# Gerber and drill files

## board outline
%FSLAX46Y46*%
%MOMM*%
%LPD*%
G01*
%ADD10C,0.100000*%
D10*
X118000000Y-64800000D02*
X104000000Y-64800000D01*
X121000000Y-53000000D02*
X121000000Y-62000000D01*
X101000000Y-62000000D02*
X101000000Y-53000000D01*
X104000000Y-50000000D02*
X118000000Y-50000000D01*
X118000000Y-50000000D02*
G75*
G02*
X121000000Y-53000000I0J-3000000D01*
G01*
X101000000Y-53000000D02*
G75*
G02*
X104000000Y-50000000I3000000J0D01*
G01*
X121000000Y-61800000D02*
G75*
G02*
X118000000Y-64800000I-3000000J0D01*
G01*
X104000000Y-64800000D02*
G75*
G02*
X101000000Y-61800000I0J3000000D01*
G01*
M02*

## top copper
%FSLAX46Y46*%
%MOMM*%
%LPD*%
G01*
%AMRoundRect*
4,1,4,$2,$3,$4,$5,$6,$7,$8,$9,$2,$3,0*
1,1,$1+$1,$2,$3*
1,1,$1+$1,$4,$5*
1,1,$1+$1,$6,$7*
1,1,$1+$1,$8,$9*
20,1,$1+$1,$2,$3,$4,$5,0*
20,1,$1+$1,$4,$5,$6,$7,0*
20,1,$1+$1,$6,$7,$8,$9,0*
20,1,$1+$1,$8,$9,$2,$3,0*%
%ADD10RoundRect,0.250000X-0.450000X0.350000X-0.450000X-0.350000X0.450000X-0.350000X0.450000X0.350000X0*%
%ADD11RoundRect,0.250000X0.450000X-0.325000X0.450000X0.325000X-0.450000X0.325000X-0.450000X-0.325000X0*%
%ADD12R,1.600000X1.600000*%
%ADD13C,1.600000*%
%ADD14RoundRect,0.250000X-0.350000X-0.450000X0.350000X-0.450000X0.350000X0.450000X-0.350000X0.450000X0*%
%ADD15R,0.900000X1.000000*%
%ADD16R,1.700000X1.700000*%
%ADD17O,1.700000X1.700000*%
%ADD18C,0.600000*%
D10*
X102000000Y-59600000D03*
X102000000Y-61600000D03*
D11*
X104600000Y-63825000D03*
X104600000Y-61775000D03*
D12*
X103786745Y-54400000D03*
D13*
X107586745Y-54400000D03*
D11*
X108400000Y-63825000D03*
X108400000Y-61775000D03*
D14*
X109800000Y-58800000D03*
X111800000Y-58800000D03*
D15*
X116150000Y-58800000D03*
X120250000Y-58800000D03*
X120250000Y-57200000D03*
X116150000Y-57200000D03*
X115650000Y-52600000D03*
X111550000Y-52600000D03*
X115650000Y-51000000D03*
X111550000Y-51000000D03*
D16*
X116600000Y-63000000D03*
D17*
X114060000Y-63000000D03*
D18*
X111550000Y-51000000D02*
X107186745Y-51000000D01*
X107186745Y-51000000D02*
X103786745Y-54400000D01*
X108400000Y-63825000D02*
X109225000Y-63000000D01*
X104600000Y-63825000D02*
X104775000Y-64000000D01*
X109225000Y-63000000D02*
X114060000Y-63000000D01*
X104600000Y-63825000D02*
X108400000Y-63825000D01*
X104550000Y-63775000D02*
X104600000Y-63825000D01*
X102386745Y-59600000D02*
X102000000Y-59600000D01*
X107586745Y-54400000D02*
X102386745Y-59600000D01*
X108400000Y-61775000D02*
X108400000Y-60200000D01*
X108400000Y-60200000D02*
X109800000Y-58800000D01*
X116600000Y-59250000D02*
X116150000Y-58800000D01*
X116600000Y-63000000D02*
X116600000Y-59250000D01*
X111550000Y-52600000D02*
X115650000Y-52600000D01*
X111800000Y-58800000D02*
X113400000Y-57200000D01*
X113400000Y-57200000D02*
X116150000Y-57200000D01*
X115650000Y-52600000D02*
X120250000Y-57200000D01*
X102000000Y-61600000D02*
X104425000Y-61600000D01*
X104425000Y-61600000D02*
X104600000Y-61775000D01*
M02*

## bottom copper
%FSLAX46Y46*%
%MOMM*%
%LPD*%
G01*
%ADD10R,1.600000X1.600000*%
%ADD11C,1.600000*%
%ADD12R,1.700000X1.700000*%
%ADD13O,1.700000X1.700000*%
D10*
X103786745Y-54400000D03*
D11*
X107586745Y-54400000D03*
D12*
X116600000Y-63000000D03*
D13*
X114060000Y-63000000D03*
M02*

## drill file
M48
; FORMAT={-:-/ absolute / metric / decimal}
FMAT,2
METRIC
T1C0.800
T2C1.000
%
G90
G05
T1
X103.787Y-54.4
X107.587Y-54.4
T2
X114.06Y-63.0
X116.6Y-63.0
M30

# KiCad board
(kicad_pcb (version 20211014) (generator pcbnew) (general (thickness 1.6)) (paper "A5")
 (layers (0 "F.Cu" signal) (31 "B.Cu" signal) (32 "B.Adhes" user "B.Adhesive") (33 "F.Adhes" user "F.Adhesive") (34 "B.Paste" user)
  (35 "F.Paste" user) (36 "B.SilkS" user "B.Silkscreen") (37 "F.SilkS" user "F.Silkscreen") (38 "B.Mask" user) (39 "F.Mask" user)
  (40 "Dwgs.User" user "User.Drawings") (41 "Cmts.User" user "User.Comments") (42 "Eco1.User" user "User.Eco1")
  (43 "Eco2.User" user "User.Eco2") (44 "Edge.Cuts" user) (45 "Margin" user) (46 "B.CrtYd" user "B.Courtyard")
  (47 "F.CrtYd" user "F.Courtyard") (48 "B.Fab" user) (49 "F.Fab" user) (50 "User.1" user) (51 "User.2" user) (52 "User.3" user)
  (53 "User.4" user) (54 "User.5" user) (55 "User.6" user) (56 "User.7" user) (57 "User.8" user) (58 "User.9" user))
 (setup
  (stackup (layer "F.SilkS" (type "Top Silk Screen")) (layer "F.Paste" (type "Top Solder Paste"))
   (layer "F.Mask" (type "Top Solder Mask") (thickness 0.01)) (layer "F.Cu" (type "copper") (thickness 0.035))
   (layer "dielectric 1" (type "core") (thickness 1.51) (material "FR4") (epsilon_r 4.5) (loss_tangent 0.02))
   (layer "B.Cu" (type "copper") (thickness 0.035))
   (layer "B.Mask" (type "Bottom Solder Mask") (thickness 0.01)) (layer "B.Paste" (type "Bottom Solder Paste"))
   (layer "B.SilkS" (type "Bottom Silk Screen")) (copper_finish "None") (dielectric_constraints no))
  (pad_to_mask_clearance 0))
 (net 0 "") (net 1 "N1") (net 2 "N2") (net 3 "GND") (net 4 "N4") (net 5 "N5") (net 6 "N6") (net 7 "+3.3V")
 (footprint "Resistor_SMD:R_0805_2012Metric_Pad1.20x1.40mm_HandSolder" (layer "F.Cu") (at 102 60.6 -90)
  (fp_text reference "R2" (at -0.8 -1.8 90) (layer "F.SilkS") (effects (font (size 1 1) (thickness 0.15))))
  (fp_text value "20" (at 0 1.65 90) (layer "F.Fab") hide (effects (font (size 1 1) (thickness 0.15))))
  (pad "1" smd roundrect (at -1 0 270) (size 1.2 1.4) (layers "F.Cu" "F.Paste" "F.Mask") (roundrect_rratio 0.208333) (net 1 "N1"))
  (pad "2" smd roundrect (at 1 0 270) (size 1.2 1.4) (layers "F.Cu" "F.Paste" "F.Mask") (roundrect_rratio 0.208333) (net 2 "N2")))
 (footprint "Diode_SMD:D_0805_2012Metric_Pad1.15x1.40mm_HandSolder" (layer "F.Cu") (at 104.6 62.8 90)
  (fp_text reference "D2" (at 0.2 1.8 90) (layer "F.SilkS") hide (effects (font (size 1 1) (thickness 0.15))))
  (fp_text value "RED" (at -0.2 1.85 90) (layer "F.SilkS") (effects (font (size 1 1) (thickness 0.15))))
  (pad "1" smd roundrect (at -1.025 0 90) (size 1.15 1.4) (layers "F.Cu" "F.Paste" "F.Mask") (roundrect_rratio 0.217391) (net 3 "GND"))
  (pad "2" smd roundrect (at 1.025 0 90) (size 1.15 1.4) (layers "F.Cu" "F.Paste" "F.Mask") (roundrect_rratio 0.217391) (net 2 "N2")))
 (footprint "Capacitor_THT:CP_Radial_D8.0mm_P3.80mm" (layer "F.Cu") (at 103.786745 54.4)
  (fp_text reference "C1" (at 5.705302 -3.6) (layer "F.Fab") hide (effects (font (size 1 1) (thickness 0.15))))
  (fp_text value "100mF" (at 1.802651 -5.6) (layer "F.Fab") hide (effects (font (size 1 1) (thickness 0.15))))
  (pad "1" thru_hole rect (at 0 0) (size 1.6 1.6) (drill 0.8) (layers *.Cu *.Mask) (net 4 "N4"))
  (pad "2" thru_hole circle (at 3.8 0) (size 1.6 1.6) (drill 0.8) (layers *.Cu *.Mask) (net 1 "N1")))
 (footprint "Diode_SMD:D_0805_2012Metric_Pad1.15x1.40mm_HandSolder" (layer "F.Cu") (at 108.4 62.8 90)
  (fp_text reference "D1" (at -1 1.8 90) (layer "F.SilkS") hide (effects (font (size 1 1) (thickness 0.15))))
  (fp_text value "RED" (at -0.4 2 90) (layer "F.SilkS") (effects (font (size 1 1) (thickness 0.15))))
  (pad "1" smd roundrect (at -1.025 0 90) (size 1.15 1.4) (layers "F.Cu" "F.Paste" "F.Mask") (roundrect_rratio 0.217391) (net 3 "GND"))
  (pad "2" smd roundrect (at 1.025 0 90) (size 1.15 1.4) (layers "F.Cu" "F.Paste" "F.Mask") (roundrect_rratio 0.217391) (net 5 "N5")))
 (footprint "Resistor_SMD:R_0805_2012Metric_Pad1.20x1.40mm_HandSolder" (layer "F.Cu") (at 110.8 58.8)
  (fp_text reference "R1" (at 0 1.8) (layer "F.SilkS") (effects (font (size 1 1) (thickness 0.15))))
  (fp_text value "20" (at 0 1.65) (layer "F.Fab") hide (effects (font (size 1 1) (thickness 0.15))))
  (pad "1" smd roundrect (at -1 0) (size 1.2 1.4) (layers "F.Cu" "F.Paste" "F.Mask") (roundrect_rratio 0.208333) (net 5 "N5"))
  (pad "2" smd roundrect (at 1 0) (size 1.2 1.4) (layers "F.Cu" "F.Paste" "F.Mask") (roundrect_rratio 0.208333) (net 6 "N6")))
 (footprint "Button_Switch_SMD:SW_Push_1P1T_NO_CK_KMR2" (layer "F.Cu") (at 118.2 58 180)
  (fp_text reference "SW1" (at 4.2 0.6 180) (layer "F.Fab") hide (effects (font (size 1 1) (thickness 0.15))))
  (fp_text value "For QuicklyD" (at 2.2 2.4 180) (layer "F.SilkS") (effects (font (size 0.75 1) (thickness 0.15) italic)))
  (pad "1" smd rect (at 2.05 -0.8 180) (size 0.9 1) (layers "F.Cu" "F.Paste" "F.Mask") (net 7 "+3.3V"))
  (pad "1" smd rect (at -2.05 -0.8 180) (size 0.9 1) (layers "F.Cu" "F.Paste" "F.Mask") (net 7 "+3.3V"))
  (pad "2" smd rect (at -2.05 0.8 180) (size 0.9 1) (layers "F.Cu" "F.Paste" "F.Mask") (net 6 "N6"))
  (pad "2" smd rect (at 2.05 0.8 180) (size 0.9 1) (layers "F.Cu" "F.Paste" "F.Mask") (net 6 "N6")))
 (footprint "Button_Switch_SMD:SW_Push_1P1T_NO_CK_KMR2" (layer "F.Cu") (at 113.6 51.8 180)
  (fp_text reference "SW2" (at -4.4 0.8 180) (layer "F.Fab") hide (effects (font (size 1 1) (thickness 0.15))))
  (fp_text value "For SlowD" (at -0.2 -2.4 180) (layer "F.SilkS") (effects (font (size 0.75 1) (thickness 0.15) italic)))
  (pad "1" smd rect (at -2.05 -0.8 180) (size 0.9 1) (layers "F.Cu" "F.Paste" "F.Mask") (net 6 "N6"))
  (pad "1" smd rect (at 2.05 -0.8 180) (size 0.9 1) (layers "F.Cu" "F.Paste" "F.Mask") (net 6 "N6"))
  (pad "2" smd rect (at -2.05 0.8 180) (size 0.9 1) (layers "F.Cu" "F.Paste" "F.Mask") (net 4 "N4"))
  (pad "2" smd rect (at 2.05 0.8 180) (size 0.9 1) (layers "F.Cu" "F.Paste" "F.Mask") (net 4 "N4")))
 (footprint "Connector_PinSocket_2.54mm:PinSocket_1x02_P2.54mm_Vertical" (layer "F.Cu") (at 116.6 63 -90)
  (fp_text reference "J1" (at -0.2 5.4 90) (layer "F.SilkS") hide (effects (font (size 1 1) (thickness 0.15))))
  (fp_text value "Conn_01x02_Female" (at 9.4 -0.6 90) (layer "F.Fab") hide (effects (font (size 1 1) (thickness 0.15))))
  (pad "1" thru_hole rect (at 0 0 270) (size 1.7 1.7) (drill 1) (layers *.Cu *.Mask) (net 7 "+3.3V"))
  (pad "2" thru_hole oval (at 0 2.54 270) (size 1.7 1.7) (drill 1) (layers *.Cu *.Mask) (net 3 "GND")))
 (gr_line (start 118 64.8) (end 104 64.8) (layer "Edge.Cuts") (width 0.1))
 (gr_line (start 121 53) (end 121 62) (layer "Edge.Cuts") (width 0.1))
 (gr_line (start 101 62) (end 101 53) (layer "Edge.Cuts") (width 0.1))
 (gr_line (start 104 50) (end 118 50) (layer "Edge.Cuts") (width 0.1))
 (gr_arc (start 118 50) (mid 120.12132 50.87868) (end 121 53) (layer "Edge.Cuts") (width 0.1))
 (gr_arc (start 101 53) (mid 101.87868 50.87868) (end 104 50) (layer "Edge.Cuts") (width 0.1))
 (gr_arc (start 121 61.8) (mid 120.12132 63.92132) (end 118 64.8) (layer "Edge.Cuts") (width 0.1))
 (gr_arc (start 104 64.8) (mid 101.87868 63.92132) (end 101 61.8) (layer "Edge.Cuts") (width 0.1))
 (segment (start 111.55 51) (end 107.186745 51) (width 0.6) (layer "F.Cu") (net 4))
 (segment (start 107.186745 51) (end 103.786745 54.4) (width 0.6) (layer "F.Cu") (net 4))
 (segment (start 108.4 63.825) (end 109.225 63) (width 0.6) (layer "F.Cu") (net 3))
 (segment (start 104.6 63.825) (end 104.775 64) (width 0.6) (layer "F.Cu") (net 3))
 (segment (start 109.225 63) (end 114.06 63) (width 0.6) (layer "F.Cu") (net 3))
 (segment (start 104.6 63.825) (end 108.4 63.825) (width 0.6) (layer "F.Cu") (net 3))
 (segment (start 104.55 63.775) (end 104.6 63.825) (width 0.6) (layer "F.Cu") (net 3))
 (segment (start 102.386745 59.6) (end 102 59.6) (width 0.6) (layer "F.Cu") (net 1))
 (segment (start 107.586745 54.4) (end 102.386745 59.6) (width 0.6) (layer "F.Cu") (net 1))
 (segment (start 108.4 61.775) (end 108.4 60.2) (width 0.6) (layer "F.Cu") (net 5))
 (segment (start 108.4 60.2) (end 109.8 58.8) (width 0.6) (layer "F.Cu") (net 5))
 (segment (start 116.6 59.25) (end 116.15 58.8) (width 0.6) (layer "F.Cu") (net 7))
 (segment (start 116.6 63) (end 116.6 59.25) (width 0.6) (layer "F.Cu") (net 7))
 (segment (start 111.55 52.6) (end 115.65 52.6) (width 0.6) (layer "F.Cu") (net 6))
 (segment (start 111.8 58.8) (end 113.4 57.2) (width 0.6) (layer "F.Cu") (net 6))
 (segment (start 113.4 57.2) (end 116.15 57.2) (width 0.6) (layer "F.Cu") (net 6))
 (segment (start 115.65 52.6) (end 120.25 57.2) (width 0.6) (layer "F.Cu") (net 6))
 (segment (start 102 61.6) (end 104.425 61.6) (width 0.6) (layer "F.Cu") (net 2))
 (segment (start 104.425 61.6) (end 104.6 61.775) (width 0.6) (layer "F.Cu") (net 2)))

